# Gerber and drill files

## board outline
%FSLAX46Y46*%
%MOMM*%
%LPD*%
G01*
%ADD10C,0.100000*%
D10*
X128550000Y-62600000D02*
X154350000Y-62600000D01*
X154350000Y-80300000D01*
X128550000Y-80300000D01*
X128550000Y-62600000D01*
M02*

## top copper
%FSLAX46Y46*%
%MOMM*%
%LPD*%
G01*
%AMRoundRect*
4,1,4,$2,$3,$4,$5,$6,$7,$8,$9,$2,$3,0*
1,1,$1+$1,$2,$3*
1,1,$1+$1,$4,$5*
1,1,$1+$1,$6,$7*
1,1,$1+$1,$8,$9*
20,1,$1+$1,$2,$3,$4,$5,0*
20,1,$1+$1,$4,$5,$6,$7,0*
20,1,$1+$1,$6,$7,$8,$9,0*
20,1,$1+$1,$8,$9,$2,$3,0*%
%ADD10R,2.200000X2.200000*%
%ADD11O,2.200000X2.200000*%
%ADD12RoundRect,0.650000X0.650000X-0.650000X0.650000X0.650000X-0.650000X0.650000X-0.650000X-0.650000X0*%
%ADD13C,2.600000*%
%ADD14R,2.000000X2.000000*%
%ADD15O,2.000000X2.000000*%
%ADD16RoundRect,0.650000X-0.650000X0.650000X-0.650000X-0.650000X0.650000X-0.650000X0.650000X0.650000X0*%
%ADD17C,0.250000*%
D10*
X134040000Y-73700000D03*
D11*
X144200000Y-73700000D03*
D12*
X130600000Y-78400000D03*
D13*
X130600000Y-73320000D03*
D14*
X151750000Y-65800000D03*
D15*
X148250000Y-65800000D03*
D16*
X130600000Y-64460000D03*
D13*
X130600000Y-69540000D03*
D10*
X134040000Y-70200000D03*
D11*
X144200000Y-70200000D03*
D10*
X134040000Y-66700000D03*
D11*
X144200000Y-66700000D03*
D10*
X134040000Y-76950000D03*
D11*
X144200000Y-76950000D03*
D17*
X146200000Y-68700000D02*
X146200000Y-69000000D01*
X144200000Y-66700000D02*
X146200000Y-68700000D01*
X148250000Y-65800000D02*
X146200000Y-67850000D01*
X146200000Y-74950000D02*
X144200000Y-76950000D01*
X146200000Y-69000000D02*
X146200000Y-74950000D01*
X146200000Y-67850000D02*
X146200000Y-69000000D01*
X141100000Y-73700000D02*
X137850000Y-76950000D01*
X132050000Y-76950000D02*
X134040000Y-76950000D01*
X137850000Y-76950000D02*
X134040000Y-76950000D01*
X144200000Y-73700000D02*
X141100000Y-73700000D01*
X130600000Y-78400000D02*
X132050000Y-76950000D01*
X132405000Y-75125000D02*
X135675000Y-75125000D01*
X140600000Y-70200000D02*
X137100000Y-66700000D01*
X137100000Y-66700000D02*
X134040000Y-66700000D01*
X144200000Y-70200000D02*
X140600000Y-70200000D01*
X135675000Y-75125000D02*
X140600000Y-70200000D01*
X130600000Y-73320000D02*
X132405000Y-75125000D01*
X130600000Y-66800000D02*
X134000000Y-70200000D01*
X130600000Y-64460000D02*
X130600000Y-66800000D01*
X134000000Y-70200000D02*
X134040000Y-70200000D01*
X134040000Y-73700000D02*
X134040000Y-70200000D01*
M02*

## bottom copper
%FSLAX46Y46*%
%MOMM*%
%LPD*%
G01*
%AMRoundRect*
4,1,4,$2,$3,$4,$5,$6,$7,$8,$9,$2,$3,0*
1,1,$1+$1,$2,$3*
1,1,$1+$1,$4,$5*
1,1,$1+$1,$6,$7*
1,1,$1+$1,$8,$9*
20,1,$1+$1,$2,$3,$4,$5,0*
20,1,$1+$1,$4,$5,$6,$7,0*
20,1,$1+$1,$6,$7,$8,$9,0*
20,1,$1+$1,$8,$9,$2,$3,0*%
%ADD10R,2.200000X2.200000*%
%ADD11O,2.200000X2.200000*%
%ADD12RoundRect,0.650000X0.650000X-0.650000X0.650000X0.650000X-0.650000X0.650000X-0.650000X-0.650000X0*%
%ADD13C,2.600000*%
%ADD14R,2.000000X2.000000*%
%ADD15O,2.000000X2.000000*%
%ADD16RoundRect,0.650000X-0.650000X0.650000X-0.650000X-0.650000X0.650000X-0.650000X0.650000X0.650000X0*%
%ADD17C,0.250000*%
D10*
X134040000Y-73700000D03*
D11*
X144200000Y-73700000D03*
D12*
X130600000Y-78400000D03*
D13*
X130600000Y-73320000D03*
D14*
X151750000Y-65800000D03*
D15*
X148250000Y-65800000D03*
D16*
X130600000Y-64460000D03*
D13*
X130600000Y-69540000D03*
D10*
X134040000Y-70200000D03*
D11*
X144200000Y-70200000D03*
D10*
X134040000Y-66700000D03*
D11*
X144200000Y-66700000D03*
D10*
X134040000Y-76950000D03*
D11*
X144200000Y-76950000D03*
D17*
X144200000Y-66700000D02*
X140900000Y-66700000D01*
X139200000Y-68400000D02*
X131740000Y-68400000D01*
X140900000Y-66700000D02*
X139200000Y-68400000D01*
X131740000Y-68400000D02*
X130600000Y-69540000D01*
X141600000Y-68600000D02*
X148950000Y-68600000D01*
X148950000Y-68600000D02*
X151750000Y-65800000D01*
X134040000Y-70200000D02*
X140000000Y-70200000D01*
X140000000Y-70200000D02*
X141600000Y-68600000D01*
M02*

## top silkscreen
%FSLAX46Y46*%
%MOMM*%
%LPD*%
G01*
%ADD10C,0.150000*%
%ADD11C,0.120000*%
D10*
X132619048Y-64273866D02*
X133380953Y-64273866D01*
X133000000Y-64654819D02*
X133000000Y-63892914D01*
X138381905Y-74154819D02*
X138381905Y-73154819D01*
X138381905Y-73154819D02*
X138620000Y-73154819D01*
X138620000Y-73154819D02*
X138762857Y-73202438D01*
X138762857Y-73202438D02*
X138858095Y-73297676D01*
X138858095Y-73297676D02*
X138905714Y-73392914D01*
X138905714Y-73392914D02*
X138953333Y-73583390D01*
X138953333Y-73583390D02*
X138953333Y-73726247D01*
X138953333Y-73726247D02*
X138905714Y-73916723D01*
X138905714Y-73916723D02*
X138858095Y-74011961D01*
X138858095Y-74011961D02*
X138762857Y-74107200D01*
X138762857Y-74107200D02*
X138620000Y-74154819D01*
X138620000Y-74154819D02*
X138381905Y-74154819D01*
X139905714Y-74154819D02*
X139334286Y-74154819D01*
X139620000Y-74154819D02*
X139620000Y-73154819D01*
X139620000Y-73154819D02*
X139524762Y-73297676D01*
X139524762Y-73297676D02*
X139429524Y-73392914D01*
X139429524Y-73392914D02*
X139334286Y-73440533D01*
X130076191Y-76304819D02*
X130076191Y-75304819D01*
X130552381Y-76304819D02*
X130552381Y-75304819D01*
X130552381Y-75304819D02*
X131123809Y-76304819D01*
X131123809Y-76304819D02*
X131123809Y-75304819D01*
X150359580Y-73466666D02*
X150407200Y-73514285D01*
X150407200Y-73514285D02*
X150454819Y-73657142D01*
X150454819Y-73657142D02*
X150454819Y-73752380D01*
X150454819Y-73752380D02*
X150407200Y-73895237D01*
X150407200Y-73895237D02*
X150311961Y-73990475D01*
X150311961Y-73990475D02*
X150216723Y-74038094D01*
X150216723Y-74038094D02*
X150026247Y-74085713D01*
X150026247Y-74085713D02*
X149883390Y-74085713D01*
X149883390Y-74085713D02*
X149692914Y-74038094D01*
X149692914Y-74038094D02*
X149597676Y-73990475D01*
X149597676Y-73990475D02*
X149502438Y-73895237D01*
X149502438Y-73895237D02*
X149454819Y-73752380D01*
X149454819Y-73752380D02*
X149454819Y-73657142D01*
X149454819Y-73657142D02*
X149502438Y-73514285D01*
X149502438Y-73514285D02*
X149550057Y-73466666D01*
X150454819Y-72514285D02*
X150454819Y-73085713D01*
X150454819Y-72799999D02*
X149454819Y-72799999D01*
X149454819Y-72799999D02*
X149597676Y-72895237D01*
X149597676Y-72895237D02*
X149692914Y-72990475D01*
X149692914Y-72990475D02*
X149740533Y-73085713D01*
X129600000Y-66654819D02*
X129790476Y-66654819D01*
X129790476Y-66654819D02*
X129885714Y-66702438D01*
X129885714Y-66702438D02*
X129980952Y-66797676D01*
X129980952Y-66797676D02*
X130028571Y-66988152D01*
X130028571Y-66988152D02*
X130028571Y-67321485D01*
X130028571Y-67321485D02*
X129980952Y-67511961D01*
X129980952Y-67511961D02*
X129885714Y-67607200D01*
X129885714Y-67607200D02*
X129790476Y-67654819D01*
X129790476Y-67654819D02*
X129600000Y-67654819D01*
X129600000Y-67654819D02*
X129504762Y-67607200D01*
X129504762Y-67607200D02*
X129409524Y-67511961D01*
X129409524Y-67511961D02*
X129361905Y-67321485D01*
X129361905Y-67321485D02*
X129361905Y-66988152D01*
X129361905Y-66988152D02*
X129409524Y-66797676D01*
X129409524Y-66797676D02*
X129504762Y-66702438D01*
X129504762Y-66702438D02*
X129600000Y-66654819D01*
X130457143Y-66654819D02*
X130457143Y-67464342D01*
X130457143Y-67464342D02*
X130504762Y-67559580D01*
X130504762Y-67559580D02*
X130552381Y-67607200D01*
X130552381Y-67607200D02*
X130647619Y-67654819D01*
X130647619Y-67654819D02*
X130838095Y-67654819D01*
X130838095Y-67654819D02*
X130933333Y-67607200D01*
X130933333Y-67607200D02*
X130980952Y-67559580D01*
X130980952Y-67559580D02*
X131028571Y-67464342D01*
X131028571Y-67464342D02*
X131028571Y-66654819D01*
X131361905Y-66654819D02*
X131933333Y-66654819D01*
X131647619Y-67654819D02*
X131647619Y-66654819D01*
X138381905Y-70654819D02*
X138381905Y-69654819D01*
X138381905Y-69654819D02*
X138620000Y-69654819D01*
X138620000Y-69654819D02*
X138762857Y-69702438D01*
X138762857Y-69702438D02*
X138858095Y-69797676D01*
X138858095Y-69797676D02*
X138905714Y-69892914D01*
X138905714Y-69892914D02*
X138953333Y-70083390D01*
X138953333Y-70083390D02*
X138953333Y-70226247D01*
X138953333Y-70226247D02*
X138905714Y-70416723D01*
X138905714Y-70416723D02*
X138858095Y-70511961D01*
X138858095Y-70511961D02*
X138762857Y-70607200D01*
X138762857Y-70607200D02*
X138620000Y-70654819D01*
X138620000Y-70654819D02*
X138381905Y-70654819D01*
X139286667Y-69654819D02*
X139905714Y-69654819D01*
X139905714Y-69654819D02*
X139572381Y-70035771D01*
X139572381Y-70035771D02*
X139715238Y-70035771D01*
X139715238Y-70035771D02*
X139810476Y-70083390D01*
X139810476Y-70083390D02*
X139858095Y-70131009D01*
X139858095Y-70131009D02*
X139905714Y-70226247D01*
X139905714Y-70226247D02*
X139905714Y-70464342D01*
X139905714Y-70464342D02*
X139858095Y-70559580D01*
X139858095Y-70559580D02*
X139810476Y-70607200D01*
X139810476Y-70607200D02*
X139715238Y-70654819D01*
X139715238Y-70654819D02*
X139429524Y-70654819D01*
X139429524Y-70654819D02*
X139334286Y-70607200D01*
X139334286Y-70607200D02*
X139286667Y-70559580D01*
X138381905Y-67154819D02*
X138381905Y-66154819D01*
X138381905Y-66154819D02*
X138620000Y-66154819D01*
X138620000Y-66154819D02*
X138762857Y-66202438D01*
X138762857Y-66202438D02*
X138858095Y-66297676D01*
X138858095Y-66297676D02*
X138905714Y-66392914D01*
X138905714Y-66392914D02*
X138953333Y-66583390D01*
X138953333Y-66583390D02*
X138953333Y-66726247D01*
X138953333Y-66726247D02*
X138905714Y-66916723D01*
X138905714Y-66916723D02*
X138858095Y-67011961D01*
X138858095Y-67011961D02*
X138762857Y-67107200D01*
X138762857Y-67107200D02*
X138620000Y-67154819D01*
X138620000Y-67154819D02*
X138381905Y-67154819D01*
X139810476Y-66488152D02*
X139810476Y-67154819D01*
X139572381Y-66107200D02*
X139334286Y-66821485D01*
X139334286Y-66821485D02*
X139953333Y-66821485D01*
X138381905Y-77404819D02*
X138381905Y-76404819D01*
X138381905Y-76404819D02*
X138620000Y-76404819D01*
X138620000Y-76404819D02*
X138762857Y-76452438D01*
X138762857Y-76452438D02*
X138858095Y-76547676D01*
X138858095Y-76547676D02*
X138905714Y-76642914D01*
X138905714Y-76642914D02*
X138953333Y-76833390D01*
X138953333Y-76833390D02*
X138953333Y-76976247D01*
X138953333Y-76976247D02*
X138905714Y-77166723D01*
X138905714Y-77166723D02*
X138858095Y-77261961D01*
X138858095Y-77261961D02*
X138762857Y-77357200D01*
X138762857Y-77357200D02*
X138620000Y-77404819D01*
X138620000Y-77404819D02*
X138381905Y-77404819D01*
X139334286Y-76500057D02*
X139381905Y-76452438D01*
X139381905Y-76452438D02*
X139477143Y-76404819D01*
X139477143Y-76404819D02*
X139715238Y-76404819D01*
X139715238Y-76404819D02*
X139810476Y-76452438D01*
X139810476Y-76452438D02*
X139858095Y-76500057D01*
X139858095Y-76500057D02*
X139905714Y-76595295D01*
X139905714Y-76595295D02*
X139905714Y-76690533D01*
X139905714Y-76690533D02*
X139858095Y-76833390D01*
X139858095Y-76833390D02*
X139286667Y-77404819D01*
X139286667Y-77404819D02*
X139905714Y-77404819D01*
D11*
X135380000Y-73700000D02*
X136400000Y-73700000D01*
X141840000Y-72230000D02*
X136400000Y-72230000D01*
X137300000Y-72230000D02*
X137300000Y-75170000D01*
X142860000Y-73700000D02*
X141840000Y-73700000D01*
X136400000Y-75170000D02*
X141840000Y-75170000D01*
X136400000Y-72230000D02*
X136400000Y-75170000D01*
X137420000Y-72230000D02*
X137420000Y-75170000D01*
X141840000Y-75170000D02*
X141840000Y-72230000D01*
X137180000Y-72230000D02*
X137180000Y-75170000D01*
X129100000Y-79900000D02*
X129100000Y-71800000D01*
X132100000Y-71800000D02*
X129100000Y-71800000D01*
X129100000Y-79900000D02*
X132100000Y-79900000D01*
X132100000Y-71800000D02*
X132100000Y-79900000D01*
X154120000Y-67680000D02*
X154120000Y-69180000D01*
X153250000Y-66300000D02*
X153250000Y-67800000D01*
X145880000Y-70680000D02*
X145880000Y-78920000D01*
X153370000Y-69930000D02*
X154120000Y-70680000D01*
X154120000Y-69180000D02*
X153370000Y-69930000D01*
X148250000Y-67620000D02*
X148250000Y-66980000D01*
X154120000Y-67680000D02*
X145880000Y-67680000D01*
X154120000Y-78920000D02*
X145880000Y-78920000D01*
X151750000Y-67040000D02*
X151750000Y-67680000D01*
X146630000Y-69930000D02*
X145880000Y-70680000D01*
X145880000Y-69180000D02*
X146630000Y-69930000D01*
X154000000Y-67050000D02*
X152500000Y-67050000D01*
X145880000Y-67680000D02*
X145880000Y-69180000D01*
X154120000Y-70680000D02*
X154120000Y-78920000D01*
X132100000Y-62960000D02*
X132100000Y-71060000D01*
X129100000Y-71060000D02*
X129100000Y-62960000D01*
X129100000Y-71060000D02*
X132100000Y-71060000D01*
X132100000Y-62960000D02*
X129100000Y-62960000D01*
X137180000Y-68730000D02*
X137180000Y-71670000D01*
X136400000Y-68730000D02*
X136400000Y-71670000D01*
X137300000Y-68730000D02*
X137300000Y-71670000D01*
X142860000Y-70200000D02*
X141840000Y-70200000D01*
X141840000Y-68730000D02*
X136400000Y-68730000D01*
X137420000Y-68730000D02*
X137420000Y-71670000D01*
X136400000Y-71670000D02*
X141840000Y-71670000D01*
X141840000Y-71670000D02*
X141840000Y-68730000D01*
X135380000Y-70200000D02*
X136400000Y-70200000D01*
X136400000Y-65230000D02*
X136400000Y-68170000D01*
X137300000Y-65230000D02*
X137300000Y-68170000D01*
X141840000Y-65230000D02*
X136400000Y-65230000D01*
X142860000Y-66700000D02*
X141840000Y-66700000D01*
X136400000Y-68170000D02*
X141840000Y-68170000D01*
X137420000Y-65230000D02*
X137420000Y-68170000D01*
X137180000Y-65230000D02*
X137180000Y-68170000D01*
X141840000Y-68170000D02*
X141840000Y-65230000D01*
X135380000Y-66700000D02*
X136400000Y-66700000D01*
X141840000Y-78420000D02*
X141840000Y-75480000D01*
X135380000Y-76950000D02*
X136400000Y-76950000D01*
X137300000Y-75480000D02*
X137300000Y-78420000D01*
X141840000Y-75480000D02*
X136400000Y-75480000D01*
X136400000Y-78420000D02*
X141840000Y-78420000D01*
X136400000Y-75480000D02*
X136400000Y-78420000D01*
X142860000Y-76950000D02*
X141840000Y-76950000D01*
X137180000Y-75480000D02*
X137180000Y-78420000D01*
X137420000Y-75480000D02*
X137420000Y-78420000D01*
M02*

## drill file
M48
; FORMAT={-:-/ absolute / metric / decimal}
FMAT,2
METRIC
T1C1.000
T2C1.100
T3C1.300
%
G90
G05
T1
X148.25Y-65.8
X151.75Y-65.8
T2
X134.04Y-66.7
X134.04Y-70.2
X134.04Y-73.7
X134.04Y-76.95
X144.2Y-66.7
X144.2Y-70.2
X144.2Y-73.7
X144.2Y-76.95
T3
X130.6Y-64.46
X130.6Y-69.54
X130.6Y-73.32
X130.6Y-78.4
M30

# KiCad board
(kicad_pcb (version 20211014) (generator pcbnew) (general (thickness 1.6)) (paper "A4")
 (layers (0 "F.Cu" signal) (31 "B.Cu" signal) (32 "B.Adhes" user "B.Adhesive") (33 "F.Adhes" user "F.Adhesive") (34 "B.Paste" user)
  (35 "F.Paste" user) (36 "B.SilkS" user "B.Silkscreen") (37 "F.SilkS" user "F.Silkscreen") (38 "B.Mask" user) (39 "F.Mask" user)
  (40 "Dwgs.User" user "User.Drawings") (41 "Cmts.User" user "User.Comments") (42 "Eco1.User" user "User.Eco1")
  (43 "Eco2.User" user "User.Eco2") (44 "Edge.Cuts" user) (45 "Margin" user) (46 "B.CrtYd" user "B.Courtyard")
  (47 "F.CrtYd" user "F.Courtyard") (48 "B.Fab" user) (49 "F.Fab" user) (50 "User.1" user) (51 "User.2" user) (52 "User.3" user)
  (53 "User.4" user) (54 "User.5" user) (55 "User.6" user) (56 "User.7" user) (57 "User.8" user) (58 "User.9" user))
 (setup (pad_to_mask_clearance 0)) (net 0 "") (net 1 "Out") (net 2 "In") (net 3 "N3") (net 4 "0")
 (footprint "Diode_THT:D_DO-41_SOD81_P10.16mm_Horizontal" (layer "F.Cu") (at 134.04 73.7)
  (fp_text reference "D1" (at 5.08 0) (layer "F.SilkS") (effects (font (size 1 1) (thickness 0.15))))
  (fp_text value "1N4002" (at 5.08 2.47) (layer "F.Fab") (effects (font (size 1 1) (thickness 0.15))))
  (fp_line (start 1.34 0) (end 2.36 0) (layer "F.SilkS") (width 0.12))
  (fp_line (start 7.8 -1.47) (end 2.36 -1.47) (layer "F.SilkS") (width 0.12))
  (fp_line (start 3.26 -1.47) (end 3.26 1.47) (layer "F.SilkS") (width 0.12))
  (fp_line (start 8.82 0) (end 7.8 0) (layer "F.SilkS") (width 0.12))
  (fp_line (start 2.36 1.47) (end 7.8 1.47) (layer "F.SilkS") (width 0.12))
  (fp_line (start 2.36 -1.47) (end 2.36 1.47) (layer "F.SilkS") (width 0.12))
  (fp_line (start 3.38 -1.47) (end 3.38 1.47) (layer "F.SilkS") (width 0.12))
  (fp_line (start 7.8 1.47) (end 7.8 -1.47) (layer "F.SilkS") (width 0.12))
  (fp_line (start 3.14 -1.47) (end 3.14 1.47) (layer "F.SilkS") (width 0.12))
  (pad "1" thru_hole rect (at 0 0) (size 2.2 2.2) (drill 1.1) (layers *.Cu *.Mask) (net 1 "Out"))
  (pad "2" thru_hole oval (at 10.16 0) (size 2.2 2.2) (drill 1.1) (layers *.Cu *.Mask) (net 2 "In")))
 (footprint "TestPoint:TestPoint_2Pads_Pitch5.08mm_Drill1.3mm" (layer "F.Cu") (at 130.6 78.4 90)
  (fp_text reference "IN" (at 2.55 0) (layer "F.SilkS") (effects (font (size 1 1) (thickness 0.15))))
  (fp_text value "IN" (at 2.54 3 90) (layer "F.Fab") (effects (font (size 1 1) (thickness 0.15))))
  (fp_line (start -1.5 -1.5) (end 6.6 -1.5) (layer "F.SilkS") (width 0.12))
  (fp_line (start 6.6 1.5) (end 6.6 -1.5) (layer "F.SilkS") (width 0.12))
  (fp_line (start -1.5 -1.5) (end -1.5 1.5) (layer "F.SilkS") (width 0.12))
  (fp_line (start 6.6 1.5) (end -1.5 1.5) (layer "F.SilkS") (width 0.12))
  (pad "1" thru_hole roundrect (at 0 0 90) (size 2.6 2.6) (drill 1.3) (layers *.Cu *.Mask) (roundrect_rratio 0.25) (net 2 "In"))
  (pad "2" thru_hole circle (at 5.08 0 90) (size 2.6 2.6) (drill 1.3) (layers *.Cu *.Mask) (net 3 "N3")))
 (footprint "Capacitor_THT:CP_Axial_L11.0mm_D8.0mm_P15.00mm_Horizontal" (layer "F.Cu") (at 150 65.8 -90)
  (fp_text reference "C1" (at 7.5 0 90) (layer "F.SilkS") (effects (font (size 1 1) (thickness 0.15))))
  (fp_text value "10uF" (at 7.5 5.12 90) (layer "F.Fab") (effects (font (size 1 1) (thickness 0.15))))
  (fp_line (start 1.88 -4.12) (end 3.38 -4.12) (layer "F.SilkS") (width 0.12))
  (fp_line (start 0.5 -3.25) (end 2 -3.25) (layer "F.SilkS") (width 0.12))
  (fp_line (start 4.88 4.12) (end 13.12 4.12) (layer "F.SilkS") (width 0.12))
  (fp_line (start 4.13 -3.37) (end 4.88 -4.12) (layer "F.SilkS") (width 0.12))
  (fp_line (start 3.38 -4.12) (end 4.13 -3.37) (layer "F.SilkS") (width 0.12))
  (fp_line (start 1.82 1.75) (end 1.18 1.75) (layer "F.SilkS") (width 0.12))
  (fp_line (start 1.88 -4.12) (end 1.88 4.12) (layer "F.SilkS") (width 0.12))
  (fp_line (start 13.12 -4.12) (end 13.12 4.12) (layer "F.SilkS") (width 0.12))
  (fp_line (start 1.24 -1.75) (end 1.88 -1.75) (layer "F.SilkS") (width 0.12))
  (fp_line (start 4.13 3.37) (end 4.88 4.12) (layer "F.SilkS") (width 0.12))
  (fp_line (start 3.38 4.12) (end 4.13 3.37) (layer "F.SilkS") (width 0.12))
  (fp_line (start 1.25 -4) (end 1.25 -2.5) (layer "F.SilkS") (width 0.12))
  (fp_line (start 1.88 4.12) (end 3.38 4.12) (layer "F.SilkS") (width 0.12))
  (fp_line (start 4.88 -4.12) (end 13.12 -4.12) (layer "F.SilkS") (width 0.12))
  (pad "1" thru_hole rect (at 0 -1.75 270) (size 2 2) (drill 1) (layers *.Cu *.Mask) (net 1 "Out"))
  (pad "2" thru_hole oval (at 0 1.75 270) (size 2 2) (drill 1) (layers *.Cu *.Mask) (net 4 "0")))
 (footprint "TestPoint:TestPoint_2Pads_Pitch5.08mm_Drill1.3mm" (layer "F.Cu") (at 130.6 64.46 -90)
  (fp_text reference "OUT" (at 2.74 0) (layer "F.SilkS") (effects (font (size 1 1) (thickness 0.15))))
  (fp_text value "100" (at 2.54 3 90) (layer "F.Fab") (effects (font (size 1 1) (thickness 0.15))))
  (fp_line (start -1.5 -1.5) (end 6.6 -1.5) (layer "F.SilkS") (width 0.12))
  (fp_line (start 6.6 1.5) (end -1.5 1.5) (layer "F.SilkS") (width 0.12))
  (fp_line (start 6.6 1.5) (end 6.6 -1.5) (layer "F.SilkS") (width 0.12))
  (fp_line (start -1.5 -1.5) (end -1.5 1.5) (layer "F.SilkS") (width 0.12))
  (pad "1" thru_hole roundrect (at 0 0 270) (size 2.6 2.6) (drill 1.3) (layers *.Cu *.Mask) (roundrect_rratio 0.25) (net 1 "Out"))
  (pad "2" thru_hole circle (at 5.08 0 270) (size 2.6 2.6) (drill 1.3) (layers *.Cu *.Mask) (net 4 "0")))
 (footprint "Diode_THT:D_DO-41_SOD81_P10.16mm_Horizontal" (layer "F.Cu") (at 134.04 70.2)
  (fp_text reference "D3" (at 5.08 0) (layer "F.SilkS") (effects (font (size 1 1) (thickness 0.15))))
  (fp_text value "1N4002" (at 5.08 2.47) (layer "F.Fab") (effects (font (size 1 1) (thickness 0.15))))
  (fp_line (start 3.14 -1.47) (end 3.14 1.47) (layer "F.SilkS") (width 0.12))
  (fp_line (start 2.36 -1.47) (end 2.36 1.47) (layer "F.SilkS") (width 0.12))
  (fp_line (start 3.26 -1.47) (end 3.26 1.47) (layer "F.SilkS") (width 0.12))
  (fp_line (start 8.82 0) (end 7.8 0) (layer "F.SilkS") (width 0.12))
  (fp_line (start 7.8 -1.47) (end 2.36 -1.47) (layer "F.SilkS") (width 0.12))
  (fp_line (start 3.38 -1.47) (end 3.38 1.47) (layer "F.SilkS") (width 0.12))
  (fp_line (start 2.36 1.47) (end 7.8 1.47) (layer "F.SilkS") (width 0.12))
  (fp_line (start 7.8 1.47) (end 7.8 -1.47) (layer "F.SilkS") (width 0.12))
  (fp_line (start 1.34 0) (end 2.36 0) (layer "F.SilkS") (width 0.12))
  (pad "1" thru_hole rect (at 0 0) (size 2.2 2.2) (drill 1.1) (layers *.Cu *.Mask) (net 1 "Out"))
  (pad "2" thru_hole oval (at 10.16 0) (size 2.2 2.2) (drill 1.1) (layers *.Cu *.Mask) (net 3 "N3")))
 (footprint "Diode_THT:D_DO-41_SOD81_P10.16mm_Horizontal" (layer "F.Cu") (at 134.04 66.7)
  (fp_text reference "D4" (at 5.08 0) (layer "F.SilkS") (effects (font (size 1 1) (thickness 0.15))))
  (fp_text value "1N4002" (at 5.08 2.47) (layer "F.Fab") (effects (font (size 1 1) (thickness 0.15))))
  (fp_line (start 2.36 -1.47) (end 2.36 1.47) (layer "F.SilkS") (width 0.12))
  (fp_line (start 3.26 -1.47) (end 3.26 1.47) (layer "F.SilkS") (width 0.12))
  (fp_line (start 7.8 -1.47) (end 2.36 -1.47) (layer "F.SilkS") (width 0.12))
  (fp_line (start 8.82 0) (end 7.8 0) (layer "F.SilkS") (width 0.12))
  (fp_line (start 2.36 1.47) (end 7.8 1.47) (layer "F.SilkS") (width 0.12))
  (fp_line (start 3.38 -1.47) (end 3.38 1.47) (layer "F.SilkS") (width 0.12))
  (fp_line (start 3.14 -1.47) (end 3.14 1.47) (layer "F.SilkS") (width 0.12))
  (fp_line (start 7.8 1.47) (end 7.8 -1.47) (layer "F.SilkS") (width 0.12))
  (fp_line (start 1.34 0) (end 2.36 0) (layer "F.SilkS") (width 0.12))
  (pad "1" thru_hole rect (at 0 0) (size 2.2 2.2) (drill 1.1) (layers *.Cu *.Mask) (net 3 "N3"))
  (pad "2" thru_hole oval (at 10.16 0) (size 2.2 2.2) (drill 1.1) (layers *.Cu *.Mask) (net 4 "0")))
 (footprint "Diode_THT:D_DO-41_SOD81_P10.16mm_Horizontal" (layer "F.Cu") (at 134.04 76.95)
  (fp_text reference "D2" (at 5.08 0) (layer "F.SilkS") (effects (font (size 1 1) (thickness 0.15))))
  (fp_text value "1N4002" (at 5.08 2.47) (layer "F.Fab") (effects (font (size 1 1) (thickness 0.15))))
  (fp_line (start 7.8 1.47) (end 7.8 -1.47) (layer "F.SilkS") (width 0.12))
  (fp_line (start 1.34 0) (end 2.36 0) (layer "F.SilkS") (width 0.12))
  (fp_line (start 3.26 -1.47) (end 3.26 1.47) (layer "F.SilkS") (width 0.12))
  (fp_line (start 7.8 -1.47) (end 2.36 -1.47) (layer "F.SilkS") (width 0.12))
  (fp_line (start 2.36 1.47) (end 7.8 1.47) (layer "F.SilkS") (width 0.12))
  (fp_line (start 2.36 -1.47) (end 2.36 1.47) (layer "F.SilkS") (width 0.12))
  (fp_line (start 8.82 0) (end 7.8 0) (layer "F.SilkS") (width 0.12))
  (fp_line (start 3.14 -1.47) (end 3.14 1.47) (layer "F.SilkS") (width 0.12))
  (fp_line (start 3.38 -1.47) (end 3.38 1.47) (layer "F.SilkS") (width 0.12))
  (pad "1" thru_hole rect (at 0 0) (size 2.2 2.2) (drill 1.1) (layers *.Cu *.Mask) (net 2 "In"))
  (pad "2" thru_hole oval (at 10.16 0) (size 2.2 2.2) (drill 1.1) (layers *.Cu *.Mask) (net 4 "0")))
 (gr_rect (start 154.35 62.6) (end 128.55 80.3) (layer "Edge.Cuts") (width 0.1) (fill none))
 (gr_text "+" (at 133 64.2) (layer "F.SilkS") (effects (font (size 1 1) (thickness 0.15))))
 (segment (start 146.2 68.7) (end 146.2 69) (width 0.25) (layer "F.Cu") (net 4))
 (segment (start 144.2 66.7) (end 146.2 68.7) (width 0.25) (layer "F.Cu") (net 4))
 (segment (start 148.25 65.8) (end 146.2 67.85) (width 0.25) (layer "F.Cu") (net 4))
 (segment (start 146.2 74.95) (end 144.2 76.95) (width 0.25) (layer "F.Cu") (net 4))
 (segment (start 146.2 69) (end 146.2 74.95) (width 0.25) (layer "F.Cu") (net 4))
 (segment (start 146.2 67.85) (end 146.2 69) (width 0.25) (layer "F.Cu") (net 4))
 (segment (start 144.2 66.7) (end 140.9 66.7) (width 0.25) (layer "B.Cu") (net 4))
 (segment (start 139.2 68.4) (end 131.74 68.4) (width 0.25) (layer "B.Cu") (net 4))
 (segment (start 140.9 66.7) (end 139.2 68.4) (width 0.25) (layer "B.Cu") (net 4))
 (segment (start 131.74 68.4) (end 130.6 69.54) (width 0.25) (layer "B.Cu") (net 4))
 (segment (start 141.1 73.7) (end 137.85 76.95) (width 0.25) (layer "F.Cu") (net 2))
 (segment (start 132.05 76.95) (end 134.04 76.95) (width 0.25) (layer "F.Cu") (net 2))
 (segment (start 137.85 76.95) (end 134.04 76.95) (width 0.25) (layer "F.Cu") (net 2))
 (segment (start 144.2 73.7) (end 141.1 73.7) (width 0.25) (layer "F.Cu") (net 2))
 (segment (start 130.6 78.4) (end 132.05 76.95) (width 0.25) (layer "F.Cu") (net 2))
 (segment (start 132.405 75.125) (end 135.675 75.125) (width 0.25) (layer "F.Cu") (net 3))
 (segment (start 140.6 70.2) (end 137.1 66.7) (width 0.25) (layer "F.Cu") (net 3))
 (segment (start 137.1 66.7) (end 134.04 66.7) (width 0.25) (layer "F.Cu") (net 3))
 (segment (start 144.2 70.2) (end 140.6 70.2) (width 0.25) (layer "F.Cu") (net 3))
 (segment (start 135.675 75.125) (end 140.6 70.2) (width 0.25) (layer "F.Cu") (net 3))
 (segment (start 130.6 73.32) (end 132.405 75.125) (width 0.25) (layer "F.Cu") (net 3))
 (segment (start 130.6 66.8) (end 134 70.2) (width 0.25) (layer "F.Cu") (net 1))
 (segment (start 130.6 64.46) (end 130.6 66.8) (width 0.25) (layer "F.Cu") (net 1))
 (segment (start 134 70.2) (end 134.04 70.2) (width 0.25) (layer "F.Cu") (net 1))
 (segment (start 134.04 73.7) (end 134.04 70.2) (width 0.25) (layer "F.Cu") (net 1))
 (segment (start 141.6 68.6) (end 148.95 68.6) (width 0.25) (layer "B.Cu") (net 1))
 (segment (start 148.95 68.6) (end 151.75 65.8) (width 0.25) (layer "B.Cu") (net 1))
 (segment (start 134.04 70.2) (end 140 70.2) (width 0.25) (layer "B.Cu") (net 1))
 (segment (start 140 70.2) (end 141.6 68.6) (width 0.25) (layer "B.Cu") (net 1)))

